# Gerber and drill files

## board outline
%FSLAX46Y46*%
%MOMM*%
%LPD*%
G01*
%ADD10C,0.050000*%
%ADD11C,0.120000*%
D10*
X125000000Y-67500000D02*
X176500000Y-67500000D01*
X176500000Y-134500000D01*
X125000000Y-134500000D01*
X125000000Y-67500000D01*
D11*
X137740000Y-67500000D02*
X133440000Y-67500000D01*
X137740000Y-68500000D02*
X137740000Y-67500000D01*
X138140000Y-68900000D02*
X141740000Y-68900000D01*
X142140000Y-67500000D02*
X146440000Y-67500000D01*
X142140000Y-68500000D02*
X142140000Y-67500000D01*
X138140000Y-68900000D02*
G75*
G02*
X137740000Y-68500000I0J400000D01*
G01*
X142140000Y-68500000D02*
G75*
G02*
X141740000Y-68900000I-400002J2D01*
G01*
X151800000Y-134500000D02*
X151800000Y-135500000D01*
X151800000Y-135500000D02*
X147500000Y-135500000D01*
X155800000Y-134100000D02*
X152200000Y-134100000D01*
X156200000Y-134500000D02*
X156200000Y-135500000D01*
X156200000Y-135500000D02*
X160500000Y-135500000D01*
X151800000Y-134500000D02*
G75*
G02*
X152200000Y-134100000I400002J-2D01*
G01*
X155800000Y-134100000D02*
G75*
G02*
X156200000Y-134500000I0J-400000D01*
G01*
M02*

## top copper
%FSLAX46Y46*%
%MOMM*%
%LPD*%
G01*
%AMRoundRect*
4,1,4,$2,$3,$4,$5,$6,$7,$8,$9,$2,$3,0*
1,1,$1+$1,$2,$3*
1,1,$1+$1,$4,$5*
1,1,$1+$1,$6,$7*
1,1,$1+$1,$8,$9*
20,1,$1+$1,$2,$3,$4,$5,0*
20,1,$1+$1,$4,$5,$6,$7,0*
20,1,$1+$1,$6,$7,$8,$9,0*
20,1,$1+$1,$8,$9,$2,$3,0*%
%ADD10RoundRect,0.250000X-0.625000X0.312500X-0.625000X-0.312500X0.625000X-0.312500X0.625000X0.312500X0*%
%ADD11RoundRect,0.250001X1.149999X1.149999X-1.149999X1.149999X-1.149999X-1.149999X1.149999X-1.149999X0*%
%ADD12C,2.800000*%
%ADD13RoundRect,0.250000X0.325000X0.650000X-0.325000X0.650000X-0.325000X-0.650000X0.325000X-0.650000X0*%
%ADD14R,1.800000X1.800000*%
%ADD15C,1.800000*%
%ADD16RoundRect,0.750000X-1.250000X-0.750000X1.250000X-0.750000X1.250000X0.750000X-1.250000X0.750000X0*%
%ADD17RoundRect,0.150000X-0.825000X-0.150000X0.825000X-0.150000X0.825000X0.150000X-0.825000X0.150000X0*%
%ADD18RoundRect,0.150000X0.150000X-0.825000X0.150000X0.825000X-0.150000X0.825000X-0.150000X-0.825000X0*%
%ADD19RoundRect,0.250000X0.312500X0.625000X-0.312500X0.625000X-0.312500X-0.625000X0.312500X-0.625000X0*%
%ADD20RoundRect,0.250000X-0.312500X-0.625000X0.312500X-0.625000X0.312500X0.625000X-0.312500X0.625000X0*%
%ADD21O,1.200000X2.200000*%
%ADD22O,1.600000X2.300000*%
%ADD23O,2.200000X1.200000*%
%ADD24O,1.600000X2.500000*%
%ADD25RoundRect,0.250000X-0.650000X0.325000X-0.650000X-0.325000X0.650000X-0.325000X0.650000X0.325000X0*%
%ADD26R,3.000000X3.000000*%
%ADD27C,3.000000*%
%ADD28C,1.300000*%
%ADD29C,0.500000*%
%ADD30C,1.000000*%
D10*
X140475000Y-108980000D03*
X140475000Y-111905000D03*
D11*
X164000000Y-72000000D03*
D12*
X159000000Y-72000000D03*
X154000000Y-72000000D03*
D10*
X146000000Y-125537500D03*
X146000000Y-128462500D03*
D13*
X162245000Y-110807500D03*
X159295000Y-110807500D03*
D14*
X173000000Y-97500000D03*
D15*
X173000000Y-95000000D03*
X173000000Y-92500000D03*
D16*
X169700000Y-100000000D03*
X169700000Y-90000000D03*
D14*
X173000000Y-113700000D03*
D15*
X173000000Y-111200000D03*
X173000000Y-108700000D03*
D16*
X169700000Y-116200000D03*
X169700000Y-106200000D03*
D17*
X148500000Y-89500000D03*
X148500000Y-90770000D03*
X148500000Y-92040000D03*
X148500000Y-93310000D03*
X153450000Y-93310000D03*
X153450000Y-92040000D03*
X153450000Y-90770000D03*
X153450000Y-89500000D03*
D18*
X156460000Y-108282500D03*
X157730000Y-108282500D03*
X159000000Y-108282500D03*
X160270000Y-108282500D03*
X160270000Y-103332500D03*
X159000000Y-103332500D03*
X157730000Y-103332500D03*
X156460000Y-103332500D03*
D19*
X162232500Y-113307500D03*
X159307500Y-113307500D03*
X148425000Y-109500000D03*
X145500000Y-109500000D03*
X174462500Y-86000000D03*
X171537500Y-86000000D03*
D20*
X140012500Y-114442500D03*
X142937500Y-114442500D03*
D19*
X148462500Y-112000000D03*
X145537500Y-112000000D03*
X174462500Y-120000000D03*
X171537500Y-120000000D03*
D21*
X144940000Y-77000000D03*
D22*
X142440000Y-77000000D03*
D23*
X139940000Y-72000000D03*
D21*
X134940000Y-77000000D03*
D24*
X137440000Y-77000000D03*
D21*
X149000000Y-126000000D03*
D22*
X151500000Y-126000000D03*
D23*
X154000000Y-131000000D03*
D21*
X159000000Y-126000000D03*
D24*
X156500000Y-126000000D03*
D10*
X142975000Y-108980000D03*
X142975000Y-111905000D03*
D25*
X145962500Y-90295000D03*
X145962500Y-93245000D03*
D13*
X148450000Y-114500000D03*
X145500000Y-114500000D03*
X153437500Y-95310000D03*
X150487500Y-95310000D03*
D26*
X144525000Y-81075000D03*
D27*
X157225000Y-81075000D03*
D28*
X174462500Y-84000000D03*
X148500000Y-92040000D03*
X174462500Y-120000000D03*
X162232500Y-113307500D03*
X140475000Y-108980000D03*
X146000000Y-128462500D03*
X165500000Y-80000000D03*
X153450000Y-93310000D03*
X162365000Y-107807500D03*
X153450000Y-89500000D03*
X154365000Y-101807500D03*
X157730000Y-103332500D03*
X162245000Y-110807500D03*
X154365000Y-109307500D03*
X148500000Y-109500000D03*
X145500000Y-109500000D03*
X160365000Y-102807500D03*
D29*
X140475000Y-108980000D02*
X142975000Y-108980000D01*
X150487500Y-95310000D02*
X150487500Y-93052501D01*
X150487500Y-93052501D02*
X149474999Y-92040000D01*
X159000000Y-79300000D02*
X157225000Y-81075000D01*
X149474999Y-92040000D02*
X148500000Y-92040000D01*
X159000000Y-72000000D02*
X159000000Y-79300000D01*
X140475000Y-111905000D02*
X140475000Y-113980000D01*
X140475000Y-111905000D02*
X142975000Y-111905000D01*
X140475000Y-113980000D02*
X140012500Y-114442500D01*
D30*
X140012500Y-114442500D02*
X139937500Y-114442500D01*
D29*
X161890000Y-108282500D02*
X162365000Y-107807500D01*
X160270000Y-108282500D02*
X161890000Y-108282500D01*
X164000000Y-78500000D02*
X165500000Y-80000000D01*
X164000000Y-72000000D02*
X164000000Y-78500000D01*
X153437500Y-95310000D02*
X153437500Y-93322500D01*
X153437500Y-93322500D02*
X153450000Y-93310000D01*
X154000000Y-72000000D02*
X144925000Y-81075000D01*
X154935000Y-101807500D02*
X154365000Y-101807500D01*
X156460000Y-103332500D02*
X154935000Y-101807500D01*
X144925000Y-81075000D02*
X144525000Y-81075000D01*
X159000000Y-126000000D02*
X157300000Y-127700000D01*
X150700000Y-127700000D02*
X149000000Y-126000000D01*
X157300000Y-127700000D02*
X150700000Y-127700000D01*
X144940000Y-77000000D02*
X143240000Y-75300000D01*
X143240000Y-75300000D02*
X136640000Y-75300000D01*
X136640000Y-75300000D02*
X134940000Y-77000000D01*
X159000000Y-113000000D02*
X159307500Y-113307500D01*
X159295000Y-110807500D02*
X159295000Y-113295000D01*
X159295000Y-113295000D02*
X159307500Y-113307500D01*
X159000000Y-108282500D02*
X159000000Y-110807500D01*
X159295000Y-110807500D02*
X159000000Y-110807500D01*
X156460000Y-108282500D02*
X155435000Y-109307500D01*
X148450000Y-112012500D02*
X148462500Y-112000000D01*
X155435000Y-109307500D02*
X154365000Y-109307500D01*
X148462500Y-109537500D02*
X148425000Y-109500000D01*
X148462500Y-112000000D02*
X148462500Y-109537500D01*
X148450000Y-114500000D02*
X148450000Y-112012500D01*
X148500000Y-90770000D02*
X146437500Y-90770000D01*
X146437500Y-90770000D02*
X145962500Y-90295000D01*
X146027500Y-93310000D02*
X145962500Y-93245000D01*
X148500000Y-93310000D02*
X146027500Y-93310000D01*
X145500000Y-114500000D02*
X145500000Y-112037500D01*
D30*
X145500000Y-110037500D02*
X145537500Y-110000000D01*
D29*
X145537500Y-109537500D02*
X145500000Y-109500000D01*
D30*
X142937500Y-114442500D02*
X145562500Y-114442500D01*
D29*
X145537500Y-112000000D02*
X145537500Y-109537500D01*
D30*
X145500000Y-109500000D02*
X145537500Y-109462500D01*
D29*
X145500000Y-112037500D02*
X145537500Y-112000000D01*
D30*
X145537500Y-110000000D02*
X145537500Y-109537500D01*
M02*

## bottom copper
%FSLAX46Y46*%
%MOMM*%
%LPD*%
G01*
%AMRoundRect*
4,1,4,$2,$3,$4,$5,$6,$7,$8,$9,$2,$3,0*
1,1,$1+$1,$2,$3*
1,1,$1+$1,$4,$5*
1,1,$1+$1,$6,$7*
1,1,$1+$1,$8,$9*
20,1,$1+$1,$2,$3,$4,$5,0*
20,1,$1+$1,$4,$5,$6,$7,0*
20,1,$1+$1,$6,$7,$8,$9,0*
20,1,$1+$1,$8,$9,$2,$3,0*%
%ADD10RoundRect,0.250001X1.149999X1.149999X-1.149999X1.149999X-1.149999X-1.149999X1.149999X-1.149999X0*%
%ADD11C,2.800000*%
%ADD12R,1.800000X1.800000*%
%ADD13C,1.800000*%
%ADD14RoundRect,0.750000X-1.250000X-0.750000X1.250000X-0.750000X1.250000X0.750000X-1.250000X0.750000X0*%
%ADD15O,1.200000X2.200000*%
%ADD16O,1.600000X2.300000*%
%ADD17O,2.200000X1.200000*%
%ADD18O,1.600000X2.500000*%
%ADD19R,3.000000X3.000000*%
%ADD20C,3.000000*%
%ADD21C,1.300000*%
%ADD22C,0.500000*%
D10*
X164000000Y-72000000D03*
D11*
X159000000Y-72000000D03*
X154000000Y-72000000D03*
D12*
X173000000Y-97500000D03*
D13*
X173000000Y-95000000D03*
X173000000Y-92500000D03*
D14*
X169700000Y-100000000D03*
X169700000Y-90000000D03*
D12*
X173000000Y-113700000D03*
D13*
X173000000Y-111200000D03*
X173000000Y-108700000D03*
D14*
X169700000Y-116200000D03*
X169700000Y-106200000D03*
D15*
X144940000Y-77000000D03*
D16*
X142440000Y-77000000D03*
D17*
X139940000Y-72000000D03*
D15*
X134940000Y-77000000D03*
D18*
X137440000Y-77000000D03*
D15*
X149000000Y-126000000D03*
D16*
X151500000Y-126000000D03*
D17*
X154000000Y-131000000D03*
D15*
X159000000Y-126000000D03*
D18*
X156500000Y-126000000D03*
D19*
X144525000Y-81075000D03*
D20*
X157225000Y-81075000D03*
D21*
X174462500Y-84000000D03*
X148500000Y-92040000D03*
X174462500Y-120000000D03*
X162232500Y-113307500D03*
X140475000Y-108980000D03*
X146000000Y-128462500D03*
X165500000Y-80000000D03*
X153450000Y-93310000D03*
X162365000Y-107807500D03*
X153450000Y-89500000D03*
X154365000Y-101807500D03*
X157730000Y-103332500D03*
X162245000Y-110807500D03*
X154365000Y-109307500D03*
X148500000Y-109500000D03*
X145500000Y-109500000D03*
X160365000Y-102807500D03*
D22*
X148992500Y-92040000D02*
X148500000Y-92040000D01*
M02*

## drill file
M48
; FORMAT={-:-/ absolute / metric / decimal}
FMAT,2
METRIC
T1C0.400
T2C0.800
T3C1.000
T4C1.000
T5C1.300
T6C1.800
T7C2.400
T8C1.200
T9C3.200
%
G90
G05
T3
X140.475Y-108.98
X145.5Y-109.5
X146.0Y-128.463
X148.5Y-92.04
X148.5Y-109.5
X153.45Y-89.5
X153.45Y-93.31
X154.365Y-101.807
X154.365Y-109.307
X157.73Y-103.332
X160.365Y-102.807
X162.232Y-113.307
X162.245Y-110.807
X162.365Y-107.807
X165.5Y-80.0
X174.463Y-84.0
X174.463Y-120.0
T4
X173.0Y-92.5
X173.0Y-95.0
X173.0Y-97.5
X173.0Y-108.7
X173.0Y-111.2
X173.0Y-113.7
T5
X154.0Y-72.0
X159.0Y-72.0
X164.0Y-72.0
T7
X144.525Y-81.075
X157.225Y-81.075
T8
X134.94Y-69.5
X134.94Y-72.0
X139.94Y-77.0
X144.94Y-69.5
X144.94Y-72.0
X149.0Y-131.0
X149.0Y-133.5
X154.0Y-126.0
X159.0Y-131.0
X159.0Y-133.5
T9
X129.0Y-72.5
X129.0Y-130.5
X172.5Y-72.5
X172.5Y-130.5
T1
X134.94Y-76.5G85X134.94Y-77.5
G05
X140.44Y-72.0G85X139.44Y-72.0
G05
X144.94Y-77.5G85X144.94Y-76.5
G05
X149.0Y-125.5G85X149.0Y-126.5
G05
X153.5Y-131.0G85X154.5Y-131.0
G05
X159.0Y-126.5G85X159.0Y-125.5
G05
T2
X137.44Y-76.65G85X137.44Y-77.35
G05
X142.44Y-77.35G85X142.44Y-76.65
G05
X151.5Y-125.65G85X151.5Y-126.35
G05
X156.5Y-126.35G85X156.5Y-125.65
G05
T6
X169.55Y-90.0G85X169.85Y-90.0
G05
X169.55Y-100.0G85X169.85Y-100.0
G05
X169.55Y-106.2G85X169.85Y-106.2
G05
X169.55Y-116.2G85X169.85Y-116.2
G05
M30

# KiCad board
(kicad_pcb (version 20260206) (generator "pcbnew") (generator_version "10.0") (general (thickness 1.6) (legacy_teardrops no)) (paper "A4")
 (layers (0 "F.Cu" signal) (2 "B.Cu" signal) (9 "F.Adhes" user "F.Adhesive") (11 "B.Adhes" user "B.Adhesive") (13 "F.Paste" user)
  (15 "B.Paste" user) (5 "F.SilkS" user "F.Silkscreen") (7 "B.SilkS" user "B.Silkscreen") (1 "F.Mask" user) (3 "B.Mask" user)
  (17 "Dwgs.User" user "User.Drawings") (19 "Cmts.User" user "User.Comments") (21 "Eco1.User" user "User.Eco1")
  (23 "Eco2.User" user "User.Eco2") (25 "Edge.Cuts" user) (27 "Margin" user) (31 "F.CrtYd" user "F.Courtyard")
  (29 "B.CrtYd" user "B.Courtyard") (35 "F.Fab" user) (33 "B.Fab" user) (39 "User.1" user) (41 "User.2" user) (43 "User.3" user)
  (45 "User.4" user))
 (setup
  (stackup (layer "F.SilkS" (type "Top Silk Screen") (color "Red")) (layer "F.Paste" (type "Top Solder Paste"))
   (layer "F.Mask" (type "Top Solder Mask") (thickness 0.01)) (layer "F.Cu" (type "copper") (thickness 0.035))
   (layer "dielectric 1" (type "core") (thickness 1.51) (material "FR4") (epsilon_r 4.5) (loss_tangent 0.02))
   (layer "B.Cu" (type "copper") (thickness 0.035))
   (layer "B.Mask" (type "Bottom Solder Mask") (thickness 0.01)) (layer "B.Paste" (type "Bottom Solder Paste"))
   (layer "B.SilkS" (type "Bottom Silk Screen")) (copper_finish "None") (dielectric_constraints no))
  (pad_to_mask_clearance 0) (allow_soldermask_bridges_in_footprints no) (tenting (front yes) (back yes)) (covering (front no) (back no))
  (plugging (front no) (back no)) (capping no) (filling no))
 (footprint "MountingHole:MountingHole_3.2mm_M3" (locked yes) (layer "F.Cu") (at 172.5 130.5)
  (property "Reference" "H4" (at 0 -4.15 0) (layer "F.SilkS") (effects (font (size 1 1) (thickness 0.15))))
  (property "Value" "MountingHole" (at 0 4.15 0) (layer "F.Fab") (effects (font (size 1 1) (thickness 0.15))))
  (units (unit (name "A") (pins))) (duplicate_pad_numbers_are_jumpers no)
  (pad "" np_thru_hole circle (at 0 0) (size 3.2 3.2) (drill 3.2) (layers "*.Cu" "*.Mask")))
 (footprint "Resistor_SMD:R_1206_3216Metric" (layer "F.Cu") (at 140.475 110.4425 -90)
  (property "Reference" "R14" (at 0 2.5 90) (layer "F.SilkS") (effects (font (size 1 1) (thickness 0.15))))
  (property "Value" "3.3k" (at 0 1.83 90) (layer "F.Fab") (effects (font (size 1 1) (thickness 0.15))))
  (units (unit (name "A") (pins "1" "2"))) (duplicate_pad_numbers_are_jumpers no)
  (pad "1" smd roundrect (at -1.4625 0 270) (size 1.125 1.75) (layers "F.Cu" "F.Mask" "F.Paste") (roundrect_rratio 0.222222) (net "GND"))
  (pad "2" smd roundrect (at 1.4625 0 270) (size 1.125 1.75) (layers "F.Cu" "F.Mask" "F.Paste") (roundrect_rratio 0.222222)
   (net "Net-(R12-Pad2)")))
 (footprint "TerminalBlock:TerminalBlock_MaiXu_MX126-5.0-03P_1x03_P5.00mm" (layer "F.Cu") (at 164 72 180)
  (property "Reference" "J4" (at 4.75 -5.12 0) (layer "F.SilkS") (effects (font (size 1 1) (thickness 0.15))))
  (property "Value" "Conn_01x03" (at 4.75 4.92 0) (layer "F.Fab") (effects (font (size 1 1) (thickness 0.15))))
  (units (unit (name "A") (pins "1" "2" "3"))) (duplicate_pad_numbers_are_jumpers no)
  (pad "1" thru_hole roundrect (at 0 0 180) (size 2.8 2.8) (drill 1.3) (layers "*.Cu" "*.Mask") (remove_unused_layers no)
   (roundrect_rratio 0.089286) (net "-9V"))
  (pad "2" thru_hole circle (at 5 0 180) (size 2.8 2.8) (drill 1.3) (layers "*.Cu" "*.Mask") (remove_unused_layers no) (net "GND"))
  (pad "3" thru_hole circle (at 10 0 180) (size 2.8 2.8) (drill 1.3) (layers "*.Cu" "*.Mask") (remove_unused_layers no) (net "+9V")))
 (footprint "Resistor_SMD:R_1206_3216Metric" (layer "F.Cu") (at 146 127 -90)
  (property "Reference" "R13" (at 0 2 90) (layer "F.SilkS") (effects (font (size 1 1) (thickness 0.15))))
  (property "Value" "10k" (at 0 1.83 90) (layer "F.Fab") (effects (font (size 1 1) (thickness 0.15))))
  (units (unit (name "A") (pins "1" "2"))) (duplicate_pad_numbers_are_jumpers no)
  (pad "1" smd roundrect (at -1.4625 0 270) (size 1.125 1.75) (layers "F.Cu" "F.Mask" "F.Paste") (roundrect_rratio 0.222222) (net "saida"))
  (pad "2" smd roundrect (at 1.4625 0 270) (size 1.125 1.75) (layers "F.Cu" "F.Mask" "F.Paste") (roundrect_rratio 0.222222) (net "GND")))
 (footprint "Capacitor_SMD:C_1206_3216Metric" (layer "F.Cu") (at 160.77 110.8075 180)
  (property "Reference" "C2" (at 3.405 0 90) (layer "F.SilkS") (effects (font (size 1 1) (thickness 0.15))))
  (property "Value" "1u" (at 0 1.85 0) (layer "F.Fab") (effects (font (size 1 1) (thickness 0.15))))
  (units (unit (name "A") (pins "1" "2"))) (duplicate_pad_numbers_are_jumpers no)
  (pad "1" smd roundrect (at -1.475 0 180) (size 1.15 1.8) (layers "F.Cu" "F.Mask" "F.Paste") (roundrect_rratio 0.217391) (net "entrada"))
  (pad "2" smd roundrect (at 1.475 0 180) (size 1.15 1.8) (layers "F.Cu" "F.Mask" "F.Paste") (roundrect_rratio 0.217391) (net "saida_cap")))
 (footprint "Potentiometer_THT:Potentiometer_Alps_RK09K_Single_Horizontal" (layer "F.Cu") (at 173 97.5 180)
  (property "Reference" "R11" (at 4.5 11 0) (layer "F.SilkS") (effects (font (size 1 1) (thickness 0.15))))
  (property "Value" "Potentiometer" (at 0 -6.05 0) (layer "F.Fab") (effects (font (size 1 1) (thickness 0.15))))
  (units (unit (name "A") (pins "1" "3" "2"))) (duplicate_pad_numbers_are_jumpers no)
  (pad "1" thru_hole rect (at 0 0) (size 1.8 1.8) (drill 1) (layers "*.Cu" "*.Mask") (remove_unused_layers no) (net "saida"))
  (pad "2" thru_hole circle (at 0 2.5) (size 1.8 1.8) (drill 1) (layers "*.Cu" "*.Mask") (remove_unused_layers no) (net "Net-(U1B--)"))
  (pad "3" thru_hole circle (at 0 5) (size 1.8 1.8) (drill 1) (layers "*.Cu" "*.Mask") (remove_unused_layers no)
   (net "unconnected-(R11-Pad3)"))
  (pad "MP" thru_hole roundrect (at 3.3 -2.5) (size 4 3) (drill oval 2.1 1.8) (layers "*.Cu" "*.Mask") (remove_unused_layers no)
   (roundrect_rratio 0.25))
  (pad "MP" thru_hole roundrect (at 3.3 7.5) (size 4 3) (drill oval 2.1 1.8) (layers "*.Cu" "*.Mask") (remove_unused_layers no)
   (roundrect_rratio 0.25))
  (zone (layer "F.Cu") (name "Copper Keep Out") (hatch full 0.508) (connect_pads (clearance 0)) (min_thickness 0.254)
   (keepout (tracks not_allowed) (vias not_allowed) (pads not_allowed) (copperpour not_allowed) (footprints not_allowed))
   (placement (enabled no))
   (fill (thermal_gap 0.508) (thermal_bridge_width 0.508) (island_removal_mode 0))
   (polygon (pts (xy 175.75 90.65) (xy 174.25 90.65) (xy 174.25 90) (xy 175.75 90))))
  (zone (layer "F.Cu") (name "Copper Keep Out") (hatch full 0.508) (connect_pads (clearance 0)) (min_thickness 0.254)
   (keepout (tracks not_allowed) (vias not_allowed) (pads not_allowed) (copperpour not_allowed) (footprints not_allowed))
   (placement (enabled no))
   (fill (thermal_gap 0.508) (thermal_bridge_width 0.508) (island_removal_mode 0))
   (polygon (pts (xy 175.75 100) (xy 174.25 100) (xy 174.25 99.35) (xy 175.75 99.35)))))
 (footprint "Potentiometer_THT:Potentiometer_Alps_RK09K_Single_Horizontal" (layer "F.Cu") (at 173 113.7 180)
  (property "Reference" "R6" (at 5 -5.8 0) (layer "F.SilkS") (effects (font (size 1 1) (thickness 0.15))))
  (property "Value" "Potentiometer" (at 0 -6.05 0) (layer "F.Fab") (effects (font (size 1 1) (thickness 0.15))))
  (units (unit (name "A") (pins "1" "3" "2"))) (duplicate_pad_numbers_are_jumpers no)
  (pad "1" thru_hole rect (at 0 0) (size 1.8 1.8) (drill 1) (layers "*.Cu" "*.Mask") (remove_unused_layers no) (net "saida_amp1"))
  (pad "2" thru_hole circle (at 0 2.5) (size 1.8 1.8) (drill 1) (layers "*.Cu" "*.Mask") (remove_unused_layers no) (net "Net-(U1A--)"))
  (pad "3" thru_hole circle (at 0 5) (size 1.8 1.8) (drill 1) (layers "*.Cu" "*.Mask") (remove_unused_layers no)
   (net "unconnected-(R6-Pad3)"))
  (pad "MP" thru_hole roundrect (at 3.3 -2.5) (size 4 3) (drill oval 2.1 1.8) (layers "*.Cu" "*.Mask") (remove_unused_layers no)
   (roundrect_rratio 0.25))
  (pad "MP" thru_hole roundrect (at 3.3 7.5) (size 4 3) (drill oval 2.1 1.8) (layers "*.Cu" "*.Mask") (remove_unused_layers no)
   (roundrect_rratio 0.25))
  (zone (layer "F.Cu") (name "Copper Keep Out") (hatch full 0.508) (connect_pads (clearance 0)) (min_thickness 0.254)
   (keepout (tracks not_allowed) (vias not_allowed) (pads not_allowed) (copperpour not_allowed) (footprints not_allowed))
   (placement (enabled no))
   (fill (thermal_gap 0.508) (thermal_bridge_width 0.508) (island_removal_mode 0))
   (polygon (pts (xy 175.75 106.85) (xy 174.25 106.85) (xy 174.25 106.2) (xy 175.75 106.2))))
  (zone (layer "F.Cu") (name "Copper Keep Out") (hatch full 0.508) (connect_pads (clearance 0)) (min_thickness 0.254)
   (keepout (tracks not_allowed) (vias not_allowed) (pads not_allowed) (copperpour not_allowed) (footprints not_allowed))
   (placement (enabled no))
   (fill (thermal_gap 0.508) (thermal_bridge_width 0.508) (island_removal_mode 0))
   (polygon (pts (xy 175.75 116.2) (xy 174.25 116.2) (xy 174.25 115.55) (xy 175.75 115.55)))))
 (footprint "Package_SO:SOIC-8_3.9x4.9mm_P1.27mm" (layer "F.Cu") (at 150.975 91.405)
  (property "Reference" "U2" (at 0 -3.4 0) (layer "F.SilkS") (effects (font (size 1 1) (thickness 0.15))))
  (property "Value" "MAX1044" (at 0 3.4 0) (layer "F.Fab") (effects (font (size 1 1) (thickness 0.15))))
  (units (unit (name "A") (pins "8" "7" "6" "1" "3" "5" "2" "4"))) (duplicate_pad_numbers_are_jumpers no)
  (pad "1" smd roundrect (at -2.475 -1.905) (size 1.95 0.6) (layers "F.Cu" "F.Mask" "F.Paste") (roundrect_rratio 0.25)
   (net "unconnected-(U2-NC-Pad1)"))
  (pad "2" smd roundrect (at -2.475 -0.635) (size 1.95 0.6) (layers "F.Cu" "F.Mask" "F.Paste") (roundrect_rratio 0.25) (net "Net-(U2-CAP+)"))
  (pad "3" smd roundrect (at -2.475 0.635) (size 1.95 0.6) (layers "F.Cu" "F.Mask" "F.Paste") (roundrect_rratio 0.25) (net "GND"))
  (pad "4" smd roundrect (at -2.475 1.905) (size 1.95 0.6) (layers "F.Cu" "F.Mask" "F.Paste") (roundrect_rratio 0.25) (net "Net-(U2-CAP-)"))
  (pad "5" smd roundrect (at 2.475 1.905) (size 1.95 0.6) (layers "F.Cu" "F.Mask" "F.Paste") (roundrect_rratio 0.25) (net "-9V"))
  (pad "6" smd roundrect (at 2.475 0.635) (size 1.95 0.6) (layers "F.Cu" "F.Mask" "F.Paste") (roundrect_rratio 0.25)
   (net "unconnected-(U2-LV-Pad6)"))
  (pad "7" smd roundrect (at 2.475 -0.635) (size 1.95 0.6) (layers "F.Cu" "F.Mask" "F.Paste") (roundrect_rratio 0.25)
   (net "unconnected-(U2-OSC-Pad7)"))
  (pad "8" smd roundrect (at 2.475 -1.905) (size 1.95 0.6) (layers "F.Cu" "F.Mask" "F.Paste") (roundrect_rratio 0.25) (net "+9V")))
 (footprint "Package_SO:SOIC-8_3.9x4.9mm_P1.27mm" (layer "F.Cu") (at 158.365 105.8075 90)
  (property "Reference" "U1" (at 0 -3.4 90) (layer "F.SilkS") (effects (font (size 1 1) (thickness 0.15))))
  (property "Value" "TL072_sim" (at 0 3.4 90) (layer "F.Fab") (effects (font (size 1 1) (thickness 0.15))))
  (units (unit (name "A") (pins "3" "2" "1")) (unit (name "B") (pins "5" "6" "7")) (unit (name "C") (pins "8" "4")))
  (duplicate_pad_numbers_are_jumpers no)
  (pad "1" smd roundrect (at -2.475 -1.905 90) (size 1.95 0.6) (layers "F.Cu" "F.Mask" "F.Paste") (roundrect_rratio 0.25) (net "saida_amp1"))
  (pad "2" smd roundrect (at -2.475 -0.635 90) (size 1.95 0.6) (layers "F.Cu" "F.Mask" "F.Paste") (roundrect_rratio 0.25)
   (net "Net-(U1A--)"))
  (pad "3" smd roundrect (at -2.475 0.635 90) (size 1.95 0.6) (layers "F.Cu" "F.Mask" "F.Paste") (roundrect_rratio 0.25) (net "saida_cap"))
  (pad "4" smd roundrect (at -2.475 1.905 90) (size 1.95 0.6) (layers "F.Cu" "F.Mask" "F.Paste") (roundrect_rratio 0.25) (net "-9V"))
  (pad "5" smd roundrect (at 2.475 1.905 90) (size 1.95 0.6) (layers "F.Cu" "F.Mask" "F.Paste") (roundrect_rratio 0.25) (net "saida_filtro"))
  (pad "6" smd roundrect (at 2.475 0.635 90) (size 1.95 0.6) (layers "F.Cu" "F.Mask" "F.Paste") (roundrect_rratio 0.25) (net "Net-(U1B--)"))
  (pad "7" smd roundrect (at 2.475 -0.635 90) (size 1.95 0.6) (layers "F.Cu" "F.Mask" "F.Paste") (roundrect_rratio 0.25) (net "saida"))
  (pad "8" smd roundrect (at 2.475 -1.905 90) (size 1.95 0.6) (layers "F.Cu" "F.Mask" "F.Paste") (roundrect_rratio 0.25) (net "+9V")))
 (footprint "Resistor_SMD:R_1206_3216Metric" (layer "F.Cu") (at 160.77 113.3075 180)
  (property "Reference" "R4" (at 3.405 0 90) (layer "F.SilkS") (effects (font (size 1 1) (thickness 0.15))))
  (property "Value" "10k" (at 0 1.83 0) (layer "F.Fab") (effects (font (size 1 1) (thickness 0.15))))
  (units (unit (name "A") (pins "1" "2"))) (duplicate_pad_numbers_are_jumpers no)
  (pad "1" smd roundrect (at -1.4625 0 180) (size 1.125 1.75) (layers "F.Cu" "F.Mask" "F.Paste") (roundrect_rratio 0.222222) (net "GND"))
  (pad "2" smd roundrect (at 1.4625 0 180) (size 1.125 1.75) (layers "F.Cu" "F.Mask" "F.Paste") (roundrect_rratio 0.222222)
   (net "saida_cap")))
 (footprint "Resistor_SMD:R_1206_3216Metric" (layer "F.Cu") (at 146.9625 109.5 180)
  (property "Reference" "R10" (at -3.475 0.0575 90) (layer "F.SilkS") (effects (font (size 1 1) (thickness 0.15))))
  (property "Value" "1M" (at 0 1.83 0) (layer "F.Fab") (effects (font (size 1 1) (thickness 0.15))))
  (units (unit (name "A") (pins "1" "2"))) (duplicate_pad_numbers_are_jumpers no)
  (pad "1" smd roundrect (at -1.4625 0 180) (size 1.125 1.75) (layers "F.Cu" "F.Mask" "F.Paste") (roundrect_rratio 0.222222)
   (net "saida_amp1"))
  (pad "2" smd roundrect (at 1.4625 0 180) (size 1.125 1.75) (layers "F.Cu" "F.Mask" "F.Paste") (roundrect_rratio 0.222222)
   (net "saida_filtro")))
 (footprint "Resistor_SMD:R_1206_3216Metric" (layer "F.Cu") (at 173 86 180)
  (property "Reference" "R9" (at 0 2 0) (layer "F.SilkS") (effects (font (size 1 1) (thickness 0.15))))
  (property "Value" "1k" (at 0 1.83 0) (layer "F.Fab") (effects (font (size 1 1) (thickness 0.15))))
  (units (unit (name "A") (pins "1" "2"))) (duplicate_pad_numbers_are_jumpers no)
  (pad "1" smd roundrect (at -1.4625 0 180) (size 1.125 1.75) (layers "F.Cu" "F.Mask" "F.Paste") (roundrect_rratio 0.222222) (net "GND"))
  (pad "2" smd roundrect (at 1.4625 0 180) (size 1.125 1.75) (layers "F.Cu" "F.Mask" "F.Paste") (roundrect_rratio 0.222222)
   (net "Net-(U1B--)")))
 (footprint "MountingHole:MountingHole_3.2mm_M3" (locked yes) (layer "F.Cu") (at 172.5 72.5)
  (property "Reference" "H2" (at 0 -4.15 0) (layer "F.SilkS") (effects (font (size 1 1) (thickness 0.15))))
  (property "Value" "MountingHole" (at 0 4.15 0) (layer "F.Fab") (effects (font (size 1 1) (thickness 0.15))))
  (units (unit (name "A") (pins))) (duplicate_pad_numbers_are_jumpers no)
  (pad "" np_thru_hole circle (at 0 0) (size 3.2 3.2) (drill 3.2) (layers "*.Cu" "*.Mask")))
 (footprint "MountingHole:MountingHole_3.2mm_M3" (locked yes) (layer "F.Cu") (at 129 72.5)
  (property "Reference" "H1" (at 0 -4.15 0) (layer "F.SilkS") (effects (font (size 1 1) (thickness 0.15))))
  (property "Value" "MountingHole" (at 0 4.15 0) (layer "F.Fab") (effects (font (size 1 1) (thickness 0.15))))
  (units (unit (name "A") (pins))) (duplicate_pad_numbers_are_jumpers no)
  (pad "" np_thru_hole circle (at 0 0) (size 3.2 3.2) (drill 3.2) (layers "*.Cu" "*.Mask")))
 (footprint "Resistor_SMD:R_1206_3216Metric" (layer "F.Cu") (at 141.475 114.4425)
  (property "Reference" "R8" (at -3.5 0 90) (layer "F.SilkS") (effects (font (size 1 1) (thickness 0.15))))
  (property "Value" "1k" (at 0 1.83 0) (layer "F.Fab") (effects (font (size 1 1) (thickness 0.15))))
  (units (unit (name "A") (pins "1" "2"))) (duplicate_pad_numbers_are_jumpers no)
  (pad "1" smd roundrect (at -1.4625 0) (size 1.125 1.75) (layers "F.Cu" "F.Mask" "F.Paste") (roundrect_rratio 0.222222)
   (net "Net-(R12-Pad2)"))
  (pad "2" smd roundrect (at 1.4625 0) (size 1.125 1.75) (layers "F.Cu" "F.Mask" "F.Paste") (roundrect_rratio 0.222222) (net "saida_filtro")))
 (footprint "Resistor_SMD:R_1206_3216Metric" (layer "F.Cu") (at 147 112 180)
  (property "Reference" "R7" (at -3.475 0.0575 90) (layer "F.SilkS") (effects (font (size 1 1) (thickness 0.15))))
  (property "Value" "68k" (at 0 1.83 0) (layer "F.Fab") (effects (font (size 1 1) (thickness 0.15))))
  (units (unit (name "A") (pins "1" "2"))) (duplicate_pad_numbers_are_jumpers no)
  (pad "1" smd roundrect (at -1.4625 0 180) (size 1.125 1.75) (layers "F.Cu" "F.Mask" "F.Paste") (roundrect_rratio 0.222222)
   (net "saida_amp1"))
  (pad "2" smd roundrect (at 1.4625 0 180) (size 1.125 1.75) (layers "F.Cu" "F.Mask" "F.Paste") (roundrect_rratio 0.222222)
   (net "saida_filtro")))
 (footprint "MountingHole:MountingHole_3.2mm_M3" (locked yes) (layer "F.Cu") (at 129 130.5)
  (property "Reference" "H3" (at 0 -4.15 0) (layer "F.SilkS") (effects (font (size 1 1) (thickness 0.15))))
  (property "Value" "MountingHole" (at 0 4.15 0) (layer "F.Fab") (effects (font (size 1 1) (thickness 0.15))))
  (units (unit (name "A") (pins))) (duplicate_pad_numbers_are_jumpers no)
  (pad "" np_thru_hole circle (at 0 0) (size 3.2 3.2) (drill 3.2) (layers "*.Cu" "*.Mask")))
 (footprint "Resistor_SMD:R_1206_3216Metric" (layer "F.Cu") (at 173 120 180)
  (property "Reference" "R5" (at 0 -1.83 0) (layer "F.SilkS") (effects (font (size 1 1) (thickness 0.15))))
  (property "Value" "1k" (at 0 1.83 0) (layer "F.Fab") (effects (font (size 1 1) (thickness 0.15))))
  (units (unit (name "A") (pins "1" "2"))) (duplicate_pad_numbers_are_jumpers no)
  (pad "1" smd roundrect (at -1.4625 0 180) (size 1.125 1.75) (layers "F.Cu" "F.Mask" "F.Paste") (roundrect_rratio 0.222222) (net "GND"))
  (pad "2" smd roundrect (at 1.4625 0 180) (size 1.125 1.75) (layers "F.Cu" "F.Mask" "F.Paste") (roundrect_rratio 0.222222)
   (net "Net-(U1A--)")))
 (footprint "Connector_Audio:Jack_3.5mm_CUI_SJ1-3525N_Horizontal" (layer "F.Cu") (at 139.94 72 180)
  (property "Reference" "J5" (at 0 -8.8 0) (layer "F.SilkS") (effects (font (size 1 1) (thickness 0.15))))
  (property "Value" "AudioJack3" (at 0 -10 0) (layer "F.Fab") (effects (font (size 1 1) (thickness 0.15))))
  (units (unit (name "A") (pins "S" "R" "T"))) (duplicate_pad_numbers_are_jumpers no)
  (fp_line (start 2.2 4.5) (end 6.5 4.5) (stroke (width 0.12) (type solid)) (layer "Edge.Cuts"))
  (fp_line (start 2.2 3.5) (end 2.2 4.5) (stroke (width 0.12) (type solid)) (layer "Edge.Cuts"))
  (fp_line (start 1.8 3.1) (end -1.8 3.1) (stroke (width 0.12) (type solid)) (layer "Edge.Cuts"))
  (fp_line (start -2.2 4.5) (end -6.5 4.5) (stroke (width 0.12) (type solid)) (layer "Edge.Cuts"))
  (fp_line (start -2.2 3.5) (end -2.2 4.5) (stroke (width 0.12) (type solid)) (layer "Edge.Cuts"))
  (fp_arc (start 1.8 3.1) (mid 2.082843 3.217157) (end 2.2 3.5) (stroke (width 0.12) (type solid)) (layer "Edge.Cuts"))
  (fp_arc (start -2.2 3.5) (mid -2.082842 3.217158) (end -1.8 3.1) (stroke (width 0.12) (type solid)) (layer "Edge.Cuts"))
  (pad "" np_thru_hole circle (at -5 0 180) (size 1.2 1.2) (drill 1.2) (layers "*.Cu" "*.Mask"))
  (pad "" np_thru_hole circle (at -5 2.5 180) (size 1.2 1.2) (drill 1.2) (layers "*.Cu" "*.Mask"))
  (pad "" np_thru_hole circle (at 0 -5 180) (size 1.2 1.2) (drill 1.2) (layers "*.Cu" "*.Mask"))
  (pad "" np_thru_hole circle (at 5 0 180) (size 1.2 1.2) (drill 1.2) (layers "*.Cu" "*.Mask"))
  (pad "" np_thru_hole circle (at 5 2.5 180) (size 1.2 1.2) (drill 1.2) (layers "*.Cu" "*.Mask"))
  (pad "R" thru_hole oval (at -5 -5 180) (size 1.2 2.2) (drill oval 0.4 1.4) (layers "*.Cu" "*.Mask") (remove_unused_layers no)
   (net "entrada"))
  (pad "RN" thru_hole oval (at -2.5 -5 180) (size 1.6 2.3) (drill oval 0.8 1.5) (layers "*.Cu" "*.Mask") (remove_unused_layers no))
  (pad "S" thru_hole oval (at 0 0 180) (size 2.2 1.2) (drill oval 1.4 0.4) (layers "*.Cu" "*.Mask") (remove_unused_layers no) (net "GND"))
  (pad "T" thru_hole oval (at 5 -5) (size 1.2 2.2) (drill oval 0.4 1.4) (layers "*.Cu" "*.Mask") (remove_unused_layers no) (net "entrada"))
  (pad "TN" thru_hole oval (at 2.5 -5) (size 1.6 2.5) (drill oval 0.8 1.5) (layers "*.Cu" "*.Mask") (remove_unused_layers no)))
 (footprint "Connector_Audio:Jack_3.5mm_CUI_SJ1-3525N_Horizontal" (layer "F.Cu") (at 154 131)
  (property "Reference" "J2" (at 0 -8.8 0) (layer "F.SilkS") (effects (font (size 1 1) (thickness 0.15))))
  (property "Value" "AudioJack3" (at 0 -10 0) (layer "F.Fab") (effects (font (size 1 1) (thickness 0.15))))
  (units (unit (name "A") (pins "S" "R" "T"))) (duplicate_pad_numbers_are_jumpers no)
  (fp_line (start -2.2 3.5) (end -2.2 4.5) (stroke (width 0.12) (type solid)) (layer "Edge.Cuts"))
  (fp_line (start -2.2 4.5) (end -6.5 4.5) (stroke (width 0.12) (type solid)) (layer "Edge.Cuts"))
  (fp_line (start 1.8 3.1) (end -1.8 3.1) (stroke (width 0.12) (type solid)) (layer "Edge.Cuts"))
  (fp_line (start 2.2 3.5) (end 2.2 4.5) (stroke (width 0.12) (type solid)) (layer "Edge.Cuts"))
  (fp_line (start 2.2 4.5) (end 6.5 4.5) (stroke (width 0.12) (type solid)) (layer "Edge.Cuts"))
  (fp_arc (start -2.2 3.5) (mid -2.082842 3.217158) (end -1.8 3.1) (stroke (width 0.12) (type solid)) (layer "Edge.Cuts"))
  (fp_arc (start 1.8 3.1) (mid 2.082843 3.217157) (end 2.2 3.5) (stroke (width 0.12) (type solid)) (layer "Edge.Cuts"))
  (pad "" np_thru_hole circle (at -5 0) (size 1.2 1.2) (drill 1.2) (layers "*.Cu" "*.Mask"))
  (pad "" np_thru_hole circle (at -5 2.5) (size 1.2 1.2) (drill 1.2) (layers "*.Cu" "*.Mask"))
  (pad "" np_thru_hole circle (at 0 -5) (size 1.2 1.2) (drill 1.2) (layers "*.Cu" "*.Mask"))
  (pad "" np_thru_hole circle (at 5 0) (size 1.2 1.2) (drill 1.2) (layers "*.Cu" "*.Mask"))
  (pad "" np_thru_hole circle (at 5 2.5) (size 1.2 1.2) (drill 1.2) (layers "*.Cu" "*.Mask"))
  (pad "R" thru_hole oval (at -5 -5) (size 1.2 2.2) (drill oval 0.4 1.4) (layers "*.Cu" "*.Mask") (remove_unused_layers no) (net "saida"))
  (pad "RN" thru_hole oval (at -2.5 -5) (size 1.6 2.3) (drill oval 0.8 1.5) (layers "*.Cu" "*.Mask") (remove_unused_layers no))
  (pad "S" thru_hole oval (at 0 0) (size 2.2 1.2) (drill oval 1.4 0.4) (layers "*.Cu" "*.Mask") (remove_unused_layers no) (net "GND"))
  (pad "T" thru_hole oval (at 5 -5 180) (size 1.2 2.2) (drill oval 0.4 1.4) (layers "*.Cu" "*.Mask") (remove_unused_layers no) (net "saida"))
  (pad "TN" thru_hole oval (at 2.5 -5 180) (size 1.6 2.5) (drill oval 0.8 1.5) (layers "*.Cu" "*.Mask") (remove_unused_layers no)))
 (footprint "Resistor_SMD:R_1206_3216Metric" (layer "F.Cu") (at 142.975 110.4425 -90)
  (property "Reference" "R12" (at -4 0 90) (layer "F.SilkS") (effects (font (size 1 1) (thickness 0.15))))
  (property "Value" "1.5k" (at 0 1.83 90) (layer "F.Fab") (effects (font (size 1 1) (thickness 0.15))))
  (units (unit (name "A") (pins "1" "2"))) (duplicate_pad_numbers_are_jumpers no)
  (pad "1" smd roundrect (at -1.4625 0 270) (size 1.125 1.75) (layers "F.Cu" "F.Mask" "F.Paste") (roundrect_rratio 0.222222) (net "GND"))
  (pad "2" smd roundrect (at 1.4625 0 270) (size 1.125 1.75) (layers "F.Cu" "F.Mask" "F.Paste") (roundrect_rratio 0.222222)
   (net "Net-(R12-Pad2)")))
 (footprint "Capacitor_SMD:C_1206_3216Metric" (layer "F.Cu") (at 145.9625 91.77 -90)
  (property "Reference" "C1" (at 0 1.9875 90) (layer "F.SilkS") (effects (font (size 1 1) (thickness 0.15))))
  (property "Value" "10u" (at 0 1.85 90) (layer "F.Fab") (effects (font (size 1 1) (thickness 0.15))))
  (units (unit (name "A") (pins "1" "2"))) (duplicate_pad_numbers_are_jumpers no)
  (pad "1" smd roundrect (at -1.475 0 270) (size 1.15 1.8) (layers "F.Cu" "F.Mask" "F.Paste") (roundrect_rratio 0.217391)
   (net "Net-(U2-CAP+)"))
  (pad "2" smd roundrect (at 1.475 0 270) (size 1.15 1.8) (layers "F.Cu" "F.Mask" "F.Paste") (roundrect_rratio 0.217391)
   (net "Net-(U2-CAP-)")))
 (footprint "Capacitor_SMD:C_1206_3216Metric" (layer "F.Cu") (at 146.975 114.5 180)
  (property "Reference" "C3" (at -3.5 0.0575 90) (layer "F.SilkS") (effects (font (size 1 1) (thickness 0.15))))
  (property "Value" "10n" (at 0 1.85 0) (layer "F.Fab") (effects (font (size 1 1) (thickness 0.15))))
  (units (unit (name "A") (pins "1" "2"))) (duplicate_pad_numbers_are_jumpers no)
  (pad "1" smd roundrect (at -1.475 0 180) (size 1.15 1.8) (layers "F.Cu" "F.Mask" "F.Paste") (roundrect_rratio 0.217391) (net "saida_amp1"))
  (pad "2" smd roundrect (at 1.475 0 180) (size 1.15 1.8) (layers "F.Cu" "F.Mask" "F.Paste") (roundrect_rratio 0.217391)
   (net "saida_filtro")))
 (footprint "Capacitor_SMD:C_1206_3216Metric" (layer "F.Cu") (at 151.9625 95.31 180)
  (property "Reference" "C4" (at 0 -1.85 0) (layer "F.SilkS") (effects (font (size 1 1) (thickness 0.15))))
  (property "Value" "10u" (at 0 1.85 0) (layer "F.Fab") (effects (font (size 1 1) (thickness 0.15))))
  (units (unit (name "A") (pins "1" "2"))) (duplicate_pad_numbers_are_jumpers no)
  (pad "1" smd roundrect (at -1.475 0 180) (size 1.15 1.8) (layers "F.Cu" "F.Mask" "F.Paste") (roundrect_rratio 0.217391) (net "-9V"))
  (pad "2" smd roundrect (at 1.475 0 180) (size 1.15 1.8) (layers "F.Cu" "F.Mask" "F.Paste") (roundrect_rratio 0.217391) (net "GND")))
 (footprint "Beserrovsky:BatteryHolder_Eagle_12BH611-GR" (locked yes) (layer "B.Cu") (at 144.525 81.075 90)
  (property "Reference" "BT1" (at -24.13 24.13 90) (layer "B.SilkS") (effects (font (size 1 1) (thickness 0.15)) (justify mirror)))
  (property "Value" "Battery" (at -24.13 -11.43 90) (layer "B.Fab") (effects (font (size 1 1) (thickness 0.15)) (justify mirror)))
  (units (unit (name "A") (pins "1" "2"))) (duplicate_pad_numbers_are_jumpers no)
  (pad "1" thru_hole rect (at 0 0 90) (size 3 3) (drill 2.4) (layers "*.Cu" "*.Mask") (remove_unused_layers no) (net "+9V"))
  (pad "2" thru_hole circle (at 0 12.7 90) (size 3 3) (drill 2.4) (layers "*.Cu" "*.Mask") (remove_unused_layers no) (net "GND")))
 (gr_rect (start 125 67.5) (end 176.5 134.5) (stroke (width 0.05) (type default)) (fill no) (locked yes) (layer "Edge.Cuts"))
 (segment (start 140.475 108.98) (end 142.975 108.98) (width 0.5) (layer "F.Cu") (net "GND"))
 (segment (start 150.4875 95.31) (end 150.4875 93.052501) (width 0.5) (layer "F.Cu") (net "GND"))
 (segment (start 150.4875 93.052501) (end 149.474999 92.04) (width 0.5) (layer "F.Cu") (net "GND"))
 (segment (start 159 79.3) (end 157.225 81.075) (width 0.5) (layer "F.Cu") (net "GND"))
 (segment (start 149.474999 92.04) (end 148.5 92.04) (width 0.5) (layer "F.Cu") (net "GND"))
 (segment (start 159 72) (end 159 79.3) (width 0.5) (layer "F.Cu") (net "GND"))
 (via (at 174.4625 84) (size 1.3) (drill 1) (layers "F.Cu" "B.Cu") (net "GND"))
 (via (at 148.5 92.04) (size 1.3) (drill 1) (layers "F.Cu" "B.Cu") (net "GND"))
 (via (at 174.4625 120) (size 1.3) (drill 1) (layers "F.Cu" "B.Cu") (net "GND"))
 (via (at 162.2325 113.3075) (size 1.3) (drill 1) (layers "F.Cu" "B.Cu") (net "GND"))
 (via (at 140.475 108.98) (size 1.3) (drill 1) (layers "F.Cu" "B.Cu") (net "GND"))
 (via (at 146 128.4625) (size 1.3) (drill 1) (layers "F.Cu" "B.Cu") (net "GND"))
 (segment (start 148.9925 92.04) (end 148.5 92.04) (width 0.5) (layer "B.Cu") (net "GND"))
 (segment (start 140.475 111.905) (end 140.475 113.98) (width 0.5) (layer "F.Cu") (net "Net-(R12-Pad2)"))
 (segment (start 140.475 111.905) (end 142.975 111.905) (width 0.5) (layer "F.Cu") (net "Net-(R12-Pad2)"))
 (segment (start 140.475 113.98) (end 140.0125 114.4425) (width 0.5) (layer "F.Cu") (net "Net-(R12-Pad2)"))
 (segment (start 140.0125 114.4425) (end 139.9375 114.4425) (width 1) (layer "F.Cu") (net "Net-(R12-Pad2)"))
 (segment (start 161.89 108.2825) (end 162.365 107.8075) (width 0.5) (layer "F.Cu") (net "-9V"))
 (segment (start 160.27 108.2825) (end 161.89 108.2825) (width 0.5) (layer "F.Cu") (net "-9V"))
 (segment (start 164 78.5) (end 165.5 80) (width 0.5) (layer "F.Cu") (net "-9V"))
 (segment (start 164 72) (end 164 78.5) (width 0.5) (layer "F.Cu") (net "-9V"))
 (segment (start 153.4375 95.31) (end 153.4375 93.3225) (width 0.5) (layer "F.Cu") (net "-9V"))
 (segment (start 153.4375 93.3225) (end 153.45 93.31) (width 0.5) (layer "F.Cu") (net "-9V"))
 (via (at 165.5 80) (size 1.3) (drill 1) (layers "F.Cu" "B.Cu") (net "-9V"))
 (via (at 153.45 93.31) (size 1.3) (drill 1) (layers "F.Cu" "B.Cu") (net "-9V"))
 (via (at 162.365 107.8075) (size 1.3) (drill 1) (layers "F.Cu" "B.Cu") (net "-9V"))
 (segment (start 154 72) (end 144.925 81.075) (width 0.5) (layer "F.Cu") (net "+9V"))
 (segment (start 154.935 101.8075) (end 154.365 101.8075) (width 0.5) (layer "F.Cu") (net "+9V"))
 (segment (start 156.46 103.3325) (end 154.935 101.8075) (width 0.5) (layer "F.Cu") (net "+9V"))
 (segment (start 144.925 81.075) (end 144.525 81.075) (width 0.5) (layer "F.Cu") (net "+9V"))
 (via (at 153.45 89.5) (size 1.3) (drill 1) (layers "F.Cu" "B.Cu") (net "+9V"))
 (via (at 154.365 101.8075) (size 1.3) (drill 1) (layers "F.Cu" "B.Cu") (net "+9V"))
 (segment (start 159 126) (end 157.3 127.7) (width 0.5) (layer "F.Cu") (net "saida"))
 (segment (start 150.7 127.7) (end 149 126) (width 0.5) (layer "F.Cu") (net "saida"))
 (segment (start 157.3 127.7) (end 150.7 127.7) (width 0.5) (layer "F.Cu") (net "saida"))
 (via (at 157.73 103.3325) (size 1.3) (drill 1) (layers "F.Cu" "B.Cu") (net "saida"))
 (segment (start 144.94 77) (end 143.24 75.3) (width 0.5) (layer "F.Cu") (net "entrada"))
 (segment (start 143.24 75.3) (end 136.64 75.3) (width 0.5) (layer "F.Cu") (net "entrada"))
 (segment (start 136.64 75.3) (end 134.94 77) (width 0.5) (layer "F.Cu") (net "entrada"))
 (via (at 162.245 110.8075) (size 1.3) (drill 1) (layers "F.Cu" "B.Cu") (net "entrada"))
 (segment (start 159 113) (end 159.3075 113.3075) (width 0.5) (layer "F.Cu") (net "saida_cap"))
 (segment (start 159.295 110.8075) (end 159.295 113.295) (width 0.5) (layer "F.Cu") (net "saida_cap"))
 (segment (start 159.295 113.295) (end 159.3075 113.3075) (width 0.5) (layer "F.Cu") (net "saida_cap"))
 (segment (start 159 108.2825) (end 159 110.8075) (width 0.5) (layer "F.Cu") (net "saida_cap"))
 (segment (start 159.295 110.8075) (end 159 110.8075) (width 0.5) (layer "F.Cu") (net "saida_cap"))
 (segment (start 156.46 108.2825) (end 155.435 109.3075) (width 0.5) (layer "F.Cu") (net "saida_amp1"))
 (segment (start 148.45 112.0125) (end 148.4625 112) (width 0.5) (layer "F.Cu") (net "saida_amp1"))
 (segment (start 155.435 109.3075) (end 154.365 109.3075) (width 0.5) (layer "F.Cu") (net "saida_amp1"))
 (segment (start 148.4625 109.5375) (end 148.425 109.5) (width 0.5) (layer "F.Cu") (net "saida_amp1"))
 (segment (start 148.4625 112) (end 148.4625 109.5375) (width 0.5) (layer "F.Cu") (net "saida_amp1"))
 (segment (start 148.45 114.5) (end 148.45 112.0125) (width 0.5) (layer "F.Cu") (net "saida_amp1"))
 (via (at 154.365 109.3075) (size 1.3) (drill 1) (layers "F.Cu" "B.Cu") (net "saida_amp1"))
 (via (at 148.5 109.5) (size 1.3) (drill 1) (layers "F.Cu" "B.Cu") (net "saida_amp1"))
 (segment (start 148.5 90.77) (end 146.4375 90.77) (width 0.5) (layer "F.Cu") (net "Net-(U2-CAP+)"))
 (segment (start 146.4375 90.77) (end 145.9625 90.295) (width 0.5) (layer "F.Cu") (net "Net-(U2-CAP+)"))
 (segment (start 146.0275 93.31) (end 145.9625 93.245) (width 0.5) (layer "F.Cu") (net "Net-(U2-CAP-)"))
 (segment (start 148.5 93.31) (end 146.0275 93.31) (width 0.5) (layer "F.Cu") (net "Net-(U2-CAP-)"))
 (segment (start 145.5 114.5) (end 145.5 112.0375) (width 0.5) (layer "F.Cu") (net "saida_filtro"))
 (segment (start 145.5 110.0375) (end 145.5375 110) (width 1) (layer "F.Cu") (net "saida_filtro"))
 (segment (start 145.5375 109.5375) (end 145.5 109.5) (width 0.5) (layer "F.Cu") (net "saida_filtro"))
 (segment (start 142.9375 114.4425) (end 145.5625 114.4425) (width 1) (layer "F.Cu") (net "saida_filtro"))
 (segment (start 145.5375 112) (end 145.5375 109.5375) (width 0.5) (layer "F.Cu") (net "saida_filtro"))
 (segment (start 145.5 109.5) (end 145.5375 109.4625) (width 1) (layer "F.Cu") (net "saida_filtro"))
 (segment (start 145.5 112.0375) (end 145.5375 112) (width 0.5) (layer "F.Cu") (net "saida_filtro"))
 (segment (start 145.5375 110) (end 145.5375 109.5375) (width 1) (layer "F.Cu") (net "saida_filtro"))
 (via (at 145.5 109.5) (size 1.3) (drill 1) (layers "F.Cu" "B.Cu") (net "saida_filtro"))
 (via (at 160.365 102.8075) (size 1.3) (drill 1) (layers "F.Cu" "B.Cu") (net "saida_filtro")))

